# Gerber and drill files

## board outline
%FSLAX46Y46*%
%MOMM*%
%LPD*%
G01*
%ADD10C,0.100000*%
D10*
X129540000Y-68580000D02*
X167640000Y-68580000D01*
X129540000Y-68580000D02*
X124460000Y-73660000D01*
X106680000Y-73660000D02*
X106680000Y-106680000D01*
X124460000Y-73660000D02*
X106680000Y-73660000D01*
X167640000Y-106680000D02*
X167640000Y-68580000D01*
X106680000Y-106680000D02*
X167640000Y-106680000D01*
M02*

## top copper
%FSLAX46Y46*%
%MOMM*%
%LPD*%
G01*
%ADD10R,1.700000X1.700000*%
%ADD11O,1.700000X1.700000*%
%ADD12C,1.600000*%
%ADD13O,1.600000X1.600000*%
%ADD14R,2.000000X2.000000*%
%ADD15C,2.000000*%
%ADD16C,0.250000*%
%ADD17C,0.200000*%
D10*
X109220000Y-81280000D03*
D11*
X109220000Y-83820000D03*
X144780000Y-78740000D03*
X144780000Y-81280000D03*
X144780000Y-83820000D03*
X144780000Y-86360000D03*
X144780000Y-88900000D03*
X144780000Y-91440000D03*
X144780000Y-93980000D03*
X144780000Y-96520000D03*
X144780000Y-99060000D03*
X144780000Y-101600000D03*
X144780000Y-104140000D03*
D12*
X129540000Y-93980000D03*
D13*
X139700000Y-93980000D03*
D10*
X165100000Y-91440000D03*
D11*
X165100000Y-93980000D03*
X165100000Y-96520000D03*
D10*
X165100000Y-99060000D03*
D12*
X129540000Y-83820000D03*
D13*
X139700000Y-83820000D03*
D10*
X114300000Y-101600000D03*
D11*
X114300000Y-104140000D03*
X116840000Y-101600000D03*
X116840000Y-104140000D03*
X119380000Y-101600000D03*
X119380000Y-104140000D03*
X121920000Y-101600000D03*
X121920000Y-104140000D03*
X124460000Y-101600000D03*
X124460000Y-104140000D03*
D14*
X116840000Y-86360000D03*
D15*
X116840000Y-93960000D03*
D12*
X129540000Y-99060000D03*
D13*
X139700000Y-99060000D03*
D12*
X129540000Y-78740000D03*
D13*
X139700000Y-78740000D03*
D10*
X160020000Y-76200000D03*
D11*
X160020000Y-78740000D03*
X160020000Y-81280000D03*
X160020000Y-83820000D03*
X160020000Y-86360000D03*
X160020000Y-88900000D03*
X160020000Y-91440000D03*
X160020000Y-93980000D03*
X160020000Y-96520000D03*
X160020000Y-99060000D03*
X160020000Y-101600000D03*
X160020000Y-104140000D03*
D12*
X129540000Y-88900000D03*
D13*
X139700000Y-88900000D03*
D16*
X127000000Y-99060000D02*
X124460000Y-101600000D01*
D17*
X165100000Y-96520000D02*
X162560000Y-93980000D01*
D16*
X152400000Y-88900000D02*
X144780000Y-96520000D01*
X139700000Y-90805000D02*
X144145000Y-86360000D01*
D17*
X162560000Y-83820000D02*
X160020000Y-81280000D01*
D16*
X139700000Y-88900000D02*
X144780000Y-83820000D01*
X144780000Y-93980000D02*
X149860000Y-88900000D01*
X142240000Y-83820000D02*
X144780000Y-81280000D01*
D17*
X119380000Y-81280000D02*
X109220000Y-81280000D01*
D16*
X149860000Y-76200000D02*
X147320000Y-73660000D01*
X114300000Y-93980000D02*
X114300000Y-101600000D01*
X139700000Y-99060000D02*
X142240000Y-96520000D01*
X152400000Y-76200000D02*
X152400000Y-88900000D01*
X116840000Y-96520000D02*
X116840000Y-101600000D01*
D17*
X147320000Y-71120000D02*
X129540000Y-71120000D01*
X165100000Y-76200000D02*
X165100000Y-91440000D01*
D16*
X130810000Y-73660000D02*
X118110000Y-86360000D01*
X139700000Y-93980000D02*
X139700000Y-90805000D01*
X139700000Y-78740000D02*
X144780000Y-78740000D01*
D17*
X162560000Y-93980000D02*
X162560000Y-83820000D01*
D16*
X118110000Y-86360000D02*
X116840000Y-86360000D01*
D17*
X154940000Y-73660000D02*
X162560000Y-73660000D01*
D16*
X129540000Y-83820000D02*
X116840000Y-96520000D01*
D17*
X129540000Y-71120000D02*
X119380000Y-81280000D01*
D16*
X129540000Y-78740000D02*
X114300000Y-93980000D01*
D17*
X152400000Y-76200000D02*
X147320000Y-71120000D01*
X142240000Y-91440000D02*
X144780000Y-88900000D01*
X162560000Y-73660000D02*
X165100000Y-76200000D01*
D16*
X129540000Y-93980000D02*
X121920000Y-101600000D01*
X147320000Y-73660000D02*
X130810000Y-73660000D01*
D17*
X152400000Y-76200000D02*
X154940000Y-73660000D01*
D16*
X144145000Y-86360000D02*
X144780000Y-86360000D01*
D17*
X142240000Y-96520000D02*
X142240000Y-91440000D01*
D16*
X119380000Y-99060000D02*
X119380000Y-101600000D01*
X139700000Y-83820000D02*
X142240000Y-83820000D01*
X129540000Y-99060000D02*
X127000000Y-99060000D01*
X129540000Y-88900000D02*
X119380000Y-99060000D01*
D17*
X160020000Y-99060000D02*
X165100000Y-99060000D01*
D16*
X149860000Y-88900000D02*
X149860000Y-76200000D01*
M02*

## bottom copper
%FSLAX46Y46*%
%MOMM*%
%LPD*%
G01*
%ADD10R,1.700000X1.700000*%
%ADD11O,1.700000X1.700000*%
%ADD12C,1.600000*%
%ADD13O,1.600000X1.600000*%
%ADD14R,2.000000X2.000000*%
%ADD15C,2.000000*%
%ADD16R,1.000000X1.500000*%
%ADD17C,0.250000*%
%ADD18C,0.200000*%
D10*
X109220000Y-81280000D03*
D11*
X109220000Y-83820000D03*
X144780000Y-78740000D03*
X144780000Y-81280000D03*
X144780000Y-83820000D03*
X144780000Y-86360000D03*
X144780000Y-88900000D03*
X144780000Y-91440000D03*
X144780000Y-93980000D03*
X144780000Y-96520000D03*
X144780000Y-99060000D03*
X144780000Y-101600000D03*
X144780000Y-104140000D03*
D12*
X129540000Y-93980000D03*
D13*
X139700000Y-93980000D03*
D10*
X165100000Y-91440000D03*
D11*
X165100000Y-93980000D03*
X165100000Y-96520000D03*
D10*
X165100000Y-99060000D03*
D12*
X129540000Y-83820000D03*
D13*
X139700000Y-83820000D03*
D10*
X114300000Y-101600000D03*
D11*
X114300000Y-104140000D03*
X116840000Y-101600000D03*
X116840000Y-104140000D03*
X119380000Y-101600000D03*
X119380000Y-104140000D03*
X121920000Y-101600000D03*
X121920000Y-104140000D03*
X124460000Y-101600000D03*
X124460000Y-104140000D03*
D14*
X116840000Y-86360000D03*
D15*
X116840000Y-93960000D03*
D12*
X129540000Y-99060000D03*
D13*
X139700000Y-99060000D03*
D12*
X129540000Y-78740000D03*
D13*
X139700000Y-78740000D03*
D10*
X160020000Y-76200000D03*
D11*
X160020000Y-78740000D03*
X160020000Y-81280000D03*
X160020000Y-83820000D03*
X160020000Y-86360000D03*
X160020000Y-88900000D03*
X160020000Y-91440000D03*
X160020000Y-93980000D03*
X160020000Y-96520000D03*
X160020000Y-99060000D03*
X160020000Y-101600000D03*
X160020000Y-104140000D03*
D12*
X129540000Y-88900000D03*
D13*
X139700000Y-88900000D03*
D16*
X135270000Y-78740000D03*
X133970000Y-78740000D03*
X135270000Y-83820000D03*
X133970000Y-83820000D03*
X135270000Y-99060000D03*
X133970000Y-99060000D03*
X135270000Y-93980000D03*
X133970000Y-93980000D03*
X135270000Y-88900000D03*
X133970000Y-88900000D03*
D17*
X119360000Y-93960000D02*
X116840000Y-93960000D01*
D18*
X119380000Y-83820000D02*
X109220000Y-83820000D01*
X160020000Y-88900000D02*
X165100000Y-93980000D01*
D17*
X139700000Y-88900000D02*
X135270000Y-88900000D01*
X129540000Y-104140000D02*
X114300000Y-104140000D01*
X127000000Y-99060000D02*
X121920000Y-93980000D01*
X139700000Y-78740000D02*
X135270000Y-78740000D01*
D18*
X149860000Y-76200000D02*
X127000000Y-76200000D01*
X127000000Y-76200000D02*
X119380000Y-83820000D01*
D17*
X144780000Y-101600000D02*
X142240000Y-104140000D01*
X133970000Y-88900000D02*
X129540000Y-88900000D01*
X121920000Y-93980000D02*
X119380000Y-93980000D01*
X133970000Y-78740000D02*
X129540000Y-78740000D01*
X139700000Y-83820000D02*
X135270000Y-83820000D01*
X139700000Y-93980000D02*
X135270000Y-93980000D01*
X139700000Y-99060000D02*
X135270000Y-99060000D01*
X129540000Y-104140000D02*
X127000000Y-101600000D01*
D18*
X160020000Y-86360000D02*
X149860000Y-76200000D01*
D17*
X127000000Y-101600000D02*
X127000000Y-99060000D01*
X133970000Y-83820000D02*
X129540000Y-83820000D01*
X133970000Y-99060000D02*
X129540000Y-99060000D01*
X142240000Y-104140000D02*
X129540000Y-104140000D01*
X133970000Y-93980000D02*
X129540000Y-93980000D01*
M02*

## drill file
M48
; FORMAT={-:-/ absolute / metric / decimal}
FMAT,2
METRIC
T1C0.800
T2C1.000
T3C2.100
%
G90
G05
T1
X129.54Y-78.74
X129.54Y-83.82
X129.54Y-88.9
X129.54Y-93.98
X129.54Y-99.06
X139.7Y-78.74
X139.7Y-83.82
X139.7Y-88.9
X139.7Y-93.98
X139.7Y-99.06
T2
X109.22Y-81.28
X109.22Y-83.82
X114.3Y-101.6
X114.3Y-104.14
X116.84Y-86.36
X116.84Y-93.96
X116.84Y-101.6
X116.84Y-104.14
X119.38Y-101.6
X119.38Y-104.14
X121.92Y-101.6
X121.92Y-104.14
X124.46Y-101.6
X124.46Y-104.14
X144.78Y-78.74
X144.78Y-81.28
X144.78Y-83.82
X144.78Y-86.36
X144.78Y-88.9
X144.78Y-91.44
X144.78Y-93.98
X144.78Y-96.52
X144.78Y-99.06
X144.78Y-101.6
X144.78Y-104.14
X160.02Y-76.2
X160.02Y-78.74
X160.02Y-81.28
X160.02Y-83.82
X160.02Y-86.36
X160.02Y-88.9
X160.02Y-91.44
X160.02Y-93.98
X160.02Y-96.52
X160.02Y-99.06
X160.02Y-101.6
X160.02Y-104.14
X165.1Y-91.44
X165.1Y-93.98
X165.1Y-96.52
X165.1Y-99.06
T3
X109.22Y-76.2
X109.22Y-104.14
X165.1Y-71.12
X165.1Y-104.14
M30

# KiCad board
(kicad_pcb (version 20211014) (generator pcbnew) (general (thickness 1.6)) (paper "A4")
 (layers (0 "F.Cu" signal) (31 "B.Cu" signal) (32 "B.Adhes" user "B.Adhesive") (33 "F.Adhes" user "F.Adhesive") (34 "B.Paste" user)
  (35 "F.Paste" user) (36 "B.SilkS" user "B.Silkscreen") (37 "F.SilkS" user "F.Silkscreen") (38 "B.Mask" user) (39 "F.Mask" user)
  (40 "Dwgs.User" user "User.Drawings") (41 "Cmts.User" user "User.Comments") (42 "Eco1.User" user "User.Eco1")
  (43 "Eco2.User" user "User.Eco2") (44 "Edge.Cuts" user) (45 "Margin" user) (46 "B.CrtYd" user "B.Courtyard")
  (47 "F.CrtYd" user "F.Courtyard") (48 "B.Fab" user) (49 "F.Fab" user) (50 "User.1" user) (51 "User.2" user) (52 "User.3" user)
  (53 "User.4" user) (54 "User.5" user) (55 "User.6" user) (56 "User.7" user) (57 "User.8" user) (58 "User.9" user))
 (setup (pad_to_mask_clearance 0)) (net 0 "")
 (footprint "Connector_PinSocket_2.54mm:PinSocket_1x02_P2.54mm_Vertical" (layer "F.Cu") (at 109.22 81.28)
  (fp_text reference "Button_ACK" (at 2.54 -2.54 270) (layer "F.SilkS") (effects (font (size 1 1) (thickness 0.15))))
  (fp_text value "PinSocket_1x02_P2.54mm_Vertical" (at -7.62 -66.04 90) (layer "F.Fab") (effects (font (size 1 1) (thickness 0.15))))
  (pad "1" thru_hole rect (at 0 0) (size 1.7 1.7) (drill 1) (layers *.Cu *.Mask))
  (pad "2" thru_hole oval (at 0 2.54) (size 1.7 1.7) (drill 1) (layers *.Cu *.Mask)))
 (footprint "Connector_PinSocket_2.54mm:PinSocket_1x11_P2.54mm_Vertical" (layer "F.Cu") (at 144.78 78.74)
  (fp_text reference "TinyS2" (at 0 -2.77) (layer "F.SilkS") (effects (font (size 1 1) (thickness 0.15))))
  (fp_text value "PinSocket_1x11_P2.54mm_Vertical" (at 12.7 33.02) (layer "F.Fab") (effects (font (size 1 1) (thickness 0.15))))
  (pad "1" thru_hole oval (at 0 0) (size 1.7 1.7) (drill 1) (layers *.Cu *.Mask))
  (pad "2" thru_hole oval (at 0 2.54) (size 1.7 1.7) (drill 1) (layers *.Cu *.Mask))
  (pad "3" thru_hole oval (at 0 5.08) (size 1.7 1.7) (drill 1) (layers *.Cu *.Mask))
  (pad "4" thru_hole oval (at 0 7.62) (size 1.7 1.7) (drill 1) (layers *.Cu *.Mask))
  (pad "5" thru_hole oval (at 0 10.16) (size 1.7 1.7) (drill 1) (layers *.Cu *.Mask))
  (pad "6" thru_hole oval (at 0 12.7) (size 1.7 1.7) (drill 1) (layers *.Cu *.Mask))
  (pad "7" thru_hole oval (at 0 15.24) (size 1.7 1.7) (drill 1) (layers *.Cu *.Mask))
  (pad "8" thru_hole oval (at 0 17.78) (size 1.7 1.7) (drill 1) (layers *.Cu *.Mask))
  (pad "9" thru_hole oval (at 0 20.32) (size 1.7 1.7) (drill 1) (layers *.Cu *.Mask))
  (pad "10" thru_hole oval (at 0 22.86) (size 1.7 1.7) (drill 1) (layers *.Cu *.Mask))
  (pad "11" thru_hole oval (at 0 25.4) (size 1.7 1.7) (drill 1) (layers *.Cu *.Mask)))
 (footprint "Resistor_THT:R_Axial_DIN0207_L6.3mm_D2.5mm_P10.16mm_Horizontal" (layer "F.Cu") (at 129.54 93.98)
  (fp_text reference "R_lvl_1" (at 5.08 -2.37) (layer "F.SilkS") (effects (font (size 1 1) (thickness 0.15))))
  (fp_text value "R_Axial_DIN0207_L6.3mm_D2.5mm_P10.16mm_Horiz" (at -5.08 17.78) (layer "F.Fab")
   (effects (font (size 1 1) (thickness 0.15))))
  (pad "1" thru_hole circle (at 0 0) (size 1.6 1.6) (drill 0.8) (layers *.Cu *.Mask))
  (pad "2" thru_hole oval (at 10.16 0) (size 1.6 1.6) (drill 0.8) (layers *.Cu *.Mask)))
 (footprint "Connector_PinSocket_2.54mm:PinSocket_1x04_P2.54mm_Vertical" (layer "F.Cu") (at 165.1 91.44)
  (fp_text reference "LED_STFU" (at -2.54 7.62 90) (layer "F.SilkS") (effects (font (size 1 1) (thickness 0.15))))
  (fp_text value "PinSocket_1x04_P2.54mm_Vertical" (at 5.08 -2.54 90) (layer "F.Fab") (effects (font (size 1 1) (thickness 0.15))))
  (pad "1" thru_hole rect (at 0 0) (size 1.7 1.7) (drill 1) (layers *.Cu *.Mask))
  (pad "2" thru_hole oval (at 0 2.54) (size 1.7 1.7) (drill 1) (layers *.Cu *.Mask))
  (pad "3" thru_hole oval (at 0 5.08) (size 1.7 1.7) (drill 1) (layers *.Cu *.Mask))
  (pad "4" thru_hole rect (at 0 7.62) (size 1.7 1.7) (drill 1) (layers *.Cu *.Mask)))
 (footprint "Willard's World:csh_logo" (layer "F.Cu") (at 116.84 78.74)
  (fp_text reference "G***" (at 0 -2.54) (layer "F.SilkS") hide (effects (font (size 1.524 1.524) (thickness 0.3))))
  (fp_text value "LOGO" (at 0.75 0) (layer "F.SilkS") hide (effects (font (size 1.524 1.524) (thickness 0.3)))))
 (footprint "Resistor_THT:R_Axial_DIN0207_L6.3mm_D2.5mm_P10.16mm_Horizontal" (layer "F.Cu") (at 129.54 83.82)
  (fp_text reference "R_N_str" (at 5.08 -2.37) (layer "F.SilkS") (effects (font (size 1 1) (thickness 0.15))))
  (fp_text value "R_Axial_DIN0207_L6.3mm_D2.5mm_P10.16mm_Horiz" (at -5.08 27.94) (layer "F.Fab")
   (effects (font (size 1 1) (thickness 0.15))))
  (pad "1" thru_hole circle (at 0 0) (size 1.6 1.6) (drill 0.8) (layers *.Cu *.Mask))
  (pad "2" thru_hole oval (at 10.16 0) (size 1.6 1.6) (drill 0.8) (layers *.Cu *.Mask)))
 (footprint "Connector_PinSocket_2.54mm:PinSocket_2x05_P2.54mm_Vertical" (layer "F.Cu") (at 114.3 101.6 90)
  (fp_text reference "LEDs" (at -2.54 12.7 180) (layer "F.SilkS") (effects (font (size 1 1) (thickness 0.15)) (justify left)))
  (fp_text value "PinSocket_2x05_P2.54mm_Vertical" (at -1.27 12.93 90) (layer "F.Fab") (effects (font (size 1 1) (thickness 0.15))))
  (pad "1" thru_hole rect (at 0 0 90) (size 1.7 1.7) (drill 1) (layers *.Cu *.Mask))
  (pad "2" thru_hole oval (at -2.54 0 90) (size 1.7 1.7) (drill 1) (layers *.Cu *.Mask))
  (pad "3" thru_hole oval (at 0 2.54 90) (size 1.7 1.7) (drill 1) (layers *.Cu *.Mask))
  (pad "4" thru_hole oval (at -2.54 2.54 90) (size 1.7 1.7) (drill 1) (layers *.Cu *.Mask))
  (pad "5" thru_hole oval (at 0 5.08 90) (size 1.7 1.7) (drill 1) (layers *.Cu *.Mask))
  (pad "6" thru_hole oval (at -2.54 5.08 90) (size 1.7 1.7) (drill 1) (layers *.Cu *.Mask))
  (pad "7" thru_hole oval (at 0 7.62 90) (size 1.7 1.7) (drill 1) (layers *.Cu *.Mask))
  (pad "8" thru_hole oval (at -2.54 7.62 90) (size 1.7 1.7) (drill 1) (layers *.Cu *.Mask))
  (pad "9" thru_hole oval (at 0 10.16 90) (size 1.7 1.7) (drill 1) (layers *.Cu *.Mask))
  (pad "10" thru_hole oval (at -2.54 10.16 90) (size 1.7 1.7) (drill 1) (layers *.Cu *.Mask)))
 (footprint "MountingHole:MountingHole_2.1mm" (layer "F.Cu") (at 109.22 76.2)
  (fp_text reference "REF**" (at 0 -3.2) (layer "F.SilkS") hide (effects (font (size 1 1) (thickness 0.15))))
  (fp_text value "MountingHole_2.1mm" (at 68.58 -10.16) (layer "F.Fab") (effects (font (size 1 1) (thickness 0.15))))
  (pad "" np_thru_hole circle (at 0 0) (size 2.1 2.1) (drill 2.1) (layers *.Cu *.Mask)))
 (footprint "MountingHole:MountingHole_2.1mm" (layer "F.Cu") (at 109.22 104.14 90)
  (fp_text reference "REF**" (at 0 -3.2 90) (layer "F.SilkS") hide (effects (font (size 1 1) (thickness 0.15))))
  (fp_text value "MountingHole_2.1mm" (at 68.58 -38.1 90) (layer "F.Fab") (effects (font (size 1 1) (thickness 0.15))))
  (pad "" np_thru_hole circle (at 0 0 90) (size 2.1 2.1) (drill 2.1) (layers *.Cu *.Mask)))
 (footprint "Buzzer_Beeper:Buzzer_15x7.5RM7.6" (layer "F.Cu") (at 116.84 86.36 -90)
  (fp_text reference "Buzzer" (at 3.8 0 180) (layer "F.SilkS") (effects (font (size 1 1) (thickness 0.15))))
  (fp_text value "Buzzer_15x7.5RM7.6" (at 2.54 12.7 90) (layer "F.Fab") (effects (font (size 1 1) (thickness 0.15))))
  (pad "1" thru_hole rect (at 0 0 270) (size 2 2) (drill 1) (layers *.Cu *.Mask))
  (pad "2" thru_hole circle (at 7.6 0 270) (size 2 2) (drill 1) (layers *.Cu *.Mask)))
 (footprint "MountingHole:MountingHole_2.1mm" (layer "F.Cu") (at 165.1 71.12)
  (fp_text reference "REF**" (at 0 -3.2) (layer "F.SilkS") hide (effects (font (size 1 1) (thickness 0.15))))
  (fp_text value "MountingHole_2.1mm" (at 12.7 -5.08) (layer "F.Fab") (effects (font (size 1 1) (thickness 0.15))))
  (pad "" np_thru_hole circle (at 0 0) (size 2.1 2.1) (drill 2.1) (layers *.Cu *.Mask)))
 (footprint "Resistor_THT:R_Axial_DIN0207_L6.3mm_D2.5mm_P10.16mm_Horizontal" (layer "F.Cu") (at 129.54 99.06)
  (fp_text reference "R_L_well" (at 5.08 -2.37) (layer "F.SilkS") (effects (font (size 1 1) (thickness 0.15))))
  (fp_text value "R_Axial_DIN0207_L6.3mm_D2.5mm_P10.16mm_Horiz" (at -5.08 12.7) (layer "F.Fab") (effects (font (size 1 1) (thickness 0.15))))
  (pad "1" thru_hole circle (at 0 0) (size 1.6 1.6) (drill 0.8) (layers *.Cu *.Mask))
  (pad "2" thru_hole oval (at 10.16 0) (size 1.6 1.6) (drill 0.8) (layers *.Cu *.Mask)))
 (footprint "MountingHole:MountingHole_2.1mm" (layer "F.Cu") (at 165.1 104.14)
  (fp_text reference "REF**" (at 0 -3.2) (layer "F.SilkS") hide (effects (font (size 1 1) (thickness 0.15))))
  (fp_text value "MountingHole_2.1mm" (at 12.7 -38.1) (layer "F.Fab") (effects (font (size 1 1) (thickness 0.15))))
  (pad "" np_thru_hole circle (at 0 0) (size 2.1 2.1) (drill 2.1) (layers *.Cu *.Mask)))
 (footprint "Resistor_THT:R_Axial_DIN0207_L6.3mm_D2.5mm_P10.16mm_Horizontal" (layer "F.Cu") (at 129.54 78.74)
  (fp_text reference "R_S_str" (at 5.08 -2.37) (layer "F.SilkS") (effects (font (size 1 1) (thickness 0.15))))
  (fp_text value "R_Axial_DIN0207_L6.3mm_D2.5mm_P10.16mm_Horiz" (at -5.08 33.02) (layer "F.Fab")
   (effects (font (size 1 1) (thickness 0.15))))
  (pad "1" thru_hole circle (at 0 0) (size 1.6 1.6) (drill 0.8) (layers *.Cu *.Mask))
  (pad "2" thru_hole oval (at 10.16 0) (size 1.6 1.6) (drill 0.8) (layers *.Cu *.Mask)))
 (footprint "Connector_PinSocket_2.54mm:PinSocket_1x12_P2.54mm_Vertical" (layer "F.Cu") (at 160.02 76.2)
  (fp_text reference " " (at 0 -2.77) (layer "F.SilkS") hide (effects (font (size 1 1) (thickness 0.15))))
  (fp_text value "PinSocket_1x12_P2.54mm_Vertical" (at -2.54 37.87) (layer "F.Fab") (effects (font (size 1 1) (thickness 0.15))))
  (pad "1" thru_hole rect (at 0 0) (size 1.7 1.7) (drill 1) (layers *.Cu *.Mask))
  (pad "2" thru_hole oval (at 0 2.54) (size 1.7 1.7) (drill 1) (layers *.Cu *.Mask))
  (pad "3" thru_hole oval (at 0 5.08) (size 1.7 1.7) (drill 1) (layers *.Cu *.Mask))
  (pad "4" thru_hole oval (at 0 7.62) (size 1.7 1.7) (drill 1) (layers *.Cu *.Mask))
  (pad "5" thru_hole oval (at 0 10.16) (size 1.7 1.7) (drill 1) (layers *.Cu *.Mask))
  (pad "6" thru_hole oval (at 0 12.7) (size 1.7 1.7) (drill 1) (layers *.Cu *.Mask))
  (pad "7" thru_hole oval (at 0 15.24) (size 1.7 1.7) (drill 1) (layers *.Cu *.Mask))
  (pad "8" thru_hole oval (at 0 17.78) (size 1.7 1.7) (drill 1) (layers *.Cu *.Mask))
  (pad "9" thru_hole oval (at 0 20.32) (size 1.7 1.7) (drill 1) (layers *.Cu *.Mask))
  (pad "10" thru_hole oval (at 0 22.86) (size 1.7 1.7) (drill 1) (layers *.Cu *.Mask))
  (pad "11" thru_hole oval (at 0 25.4) (size 1.7 1.7) (drill 1) (layers *.Cu *.Mask))
  (pad "12" thru_hole oval (at 0 27.94) (size 1.7 1.7) (drill 1) (layers *.Cu *.Mask)))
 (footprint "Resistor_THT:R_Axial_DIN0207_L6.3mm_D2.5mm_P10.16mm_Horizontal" (layer "F.Cu") (at 129.54 88.9)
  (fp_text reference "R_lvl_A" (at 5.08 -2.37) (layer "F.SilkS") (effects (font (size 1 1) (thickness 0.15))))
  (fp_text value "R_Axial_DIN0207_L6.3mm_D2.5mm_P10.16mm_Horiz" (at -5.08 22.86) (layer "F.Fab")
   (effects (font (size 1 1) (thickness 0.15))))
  (pad "1" thru_hole circle (at 0 0) (size 1.6 1.6) (drill 0.8) (layers *.Cu *.Mask))
  (pad "2" thru_hole oval (at 10.16 0) (size 1.6 1.6) (drill 0.8) (layers *.Cu *.Mask)))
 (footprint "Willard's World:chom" (layer "B.Cu") (at 116.84 93.98 180)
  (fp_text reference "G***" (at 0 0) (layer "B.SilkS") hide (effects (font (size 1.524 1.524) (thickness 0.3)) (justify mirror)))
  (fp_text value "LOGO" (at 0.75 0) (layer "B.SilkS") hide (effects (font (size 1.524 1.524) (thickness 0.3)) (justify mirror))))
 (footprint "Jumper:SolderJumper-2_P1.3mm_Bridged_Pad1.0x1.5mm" (layer "B.Cu") (at 134.62 78.74 180)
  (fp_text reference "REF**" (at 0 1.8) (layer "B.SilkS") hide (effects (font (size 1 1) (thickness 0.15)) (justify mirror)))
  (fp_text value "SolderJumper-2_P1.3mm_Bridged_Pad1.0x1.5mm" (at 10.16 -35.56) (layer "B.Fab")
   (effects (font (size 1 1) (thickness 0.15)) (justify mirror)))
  (pad "1" smd rect (at -0.65 0 180) (size 1 1.5) (layers "B.Cu" "B.Mask"))
  (pad "2" smd rect (at 0.65 0 180) (size 1 1.5) (layers "B.Cu" "B.Mask")))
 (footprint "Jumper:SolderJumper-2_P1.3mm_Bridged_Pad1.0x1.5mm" (layer "B.Cu") (at 134.62 83.82 180)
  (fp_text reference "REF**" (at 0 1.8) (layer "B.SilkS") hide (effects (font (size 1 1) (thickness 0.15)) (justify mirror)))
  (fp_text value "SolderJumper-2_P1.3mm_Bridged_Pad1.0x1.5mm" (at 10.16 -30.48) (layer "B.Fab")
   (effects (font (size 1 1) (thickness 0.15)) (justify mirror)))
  (pad "1" smd rect (at -0.65 0 180) (size 1 1.5) (layers "B.Cu" "B.Mask"))
  (pad "2" smd rect (at 0.65 0 180) (size 1 1.5) (layers "B.Cu" "B.Mask")))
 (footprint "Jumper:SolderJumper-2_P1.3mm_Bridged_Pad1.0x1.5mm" (layer "B.Cu") (at 134.62 99.06 180)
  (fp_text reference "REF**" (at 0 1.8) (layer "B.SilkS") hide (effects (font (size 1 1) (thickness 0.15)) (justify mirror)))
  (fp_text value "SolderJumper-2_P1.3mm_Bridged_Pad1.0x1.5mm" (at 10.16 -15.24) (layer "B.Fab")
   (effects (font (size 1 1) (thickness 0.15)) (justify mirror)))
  (pad "1" smd rect (at -0.65 0 180) (size 1 1.5) (layers "B.Cu" "B.Mask"))
  (pad "2" smd rect (at 0.65 0 180) (size 1 1.5) (layers "B.Cu" "B.Mask")))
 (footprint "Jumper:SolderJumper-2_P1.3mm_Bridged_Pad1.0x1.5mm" (layer "B.Cu") (at 134.62 93.98 180)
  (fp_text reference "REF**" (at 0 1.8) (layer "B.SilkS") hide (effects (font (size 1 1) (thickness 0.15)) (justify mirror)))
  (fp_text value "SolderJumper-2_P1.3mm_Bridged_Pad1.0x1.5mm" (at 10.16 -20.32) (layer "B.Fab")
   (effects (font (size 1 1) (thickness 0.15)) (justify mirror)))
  (pad "1" smd rect (at -0.65 0 180) (size 1 1.5) (layers "B.Cu" "B.Mask"))
  (pad "2" smd rect (at 0.65 0 180) (size 1 1.5) (layers "B.Cu" "B.Mask")))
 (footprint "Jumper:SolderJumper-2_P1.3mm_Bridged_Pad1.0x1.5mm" (layer "B.Cu") (at 134.62 88.9 180)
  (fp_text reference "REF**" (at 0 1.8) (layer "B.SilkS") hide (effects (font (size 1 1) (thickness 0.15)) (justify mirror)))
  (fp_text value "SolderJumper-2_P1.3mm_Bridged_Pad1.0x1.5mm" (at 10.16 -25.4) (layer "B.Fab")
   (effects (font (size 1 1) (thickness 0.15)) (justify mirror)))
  (pad "1" smd rect (at -0.65 0 180) (size 1 1.5) (layers "B.Cu" "B.Mask"))
  (pad "2" smd rect (at 0.65 0 180) (size 1 1.5) (layers "B.Cu" "B.Mask")))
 (gr_line (start 129.54 68.58) (end 167.64 68.58) (layer "Edge.Cuts") (width 0.1))
 (gr_line (start 129.54 68.58) (end 124.46 73.66) (layer "Edge.Cuts") (width 0.1))
 (gr_line (start 106.68 73.66) (end 106.68 106.68) (layer "Edge.Cuts") (width 0.1))
 (gr_line (start 124.46 73.66) (end 106.68 73.66) (layer "Edge.Cuts") (width 0.1))
 (gr_line (start 167.64 106.68) (end 167.64 68.58) (layer "Edge.Cuts") (width 0.1))
 (gr_line (start 106.68 106.68) (end 167.64 106.68) (layer "Edge.Cuts") (width 0.1))
 (segment (start 127 99.06) (end 124.46 101.6) (width 0.25) (layer "F.Cu") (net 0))
 (segment (start 165.1 96.52) (end 162.56 93.98) (width 0.2) (layer "F.Cu") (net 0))
 (segment (start 152.4 88.9) (end 144.78 96.52) (width 0.25) (layer "F.Cu") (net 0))
 (segment (start 139.7 90.805) (end 144.145 86.36) (width 0.25) (layer "F.Cu") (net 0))
 (segment (start 162.56 83.82) (end 160.02 81.28) (width 0.2) (layer "F.Cu") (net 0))
 (segment (start 139.7 88.9) (end 144.78 83.82) (width 0.25) (layer "F.Cu") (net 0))
 (segment (start 144.78 93.98) (end 149.86 88.9) (width 0.25) (layer "F.Cu") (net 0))
 (segment (start 142.24 83.82) (end 144.78 81.28) (width 0.25) (layer "F.Cu") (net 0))
 (segment (start 119.38 81.28) (end 109.22 81.28) (width 0.2) (layer "F.Cu") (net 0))
 (segment (start 149.86 76.2) (end 147.32 73.66) (width 0.25) (layer "F.Cu") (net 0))
 (segment (start 114.3 93.98) (end 114.3 101.6) (width 0.25) (layer "F.Cu") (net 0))
 (segment (start 139.7 99.06) (end 142.24 96.52) (width 0.25) (layer "F.Cu") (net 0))
 (segment (start 152.4 76.2) (end 152.4 88.9) (width 0.25) (layer "F.Cu") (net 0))
 (segment (start 116.84 96.52) (end 116.84 101.6) (width 0.25) (layer "F.Cu") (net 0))
 (segment (start 147.32 71.12) (end 129.54 71.12) (width 0.2) (layer "F.Cu") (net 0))
 (segment (start 165.1 76.2) (end 165.1 91.44) (width 0.2) (layer "F.Cu") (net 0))
 (segment (start 130.81 73.66) (end 118.11 86.36) (width 0.25) (layer "F.Cu") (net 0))
 (segment (start 139.7 93.98) (end 139.7 90.805) (width 0.25) (layer "F.Cu") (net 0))
 (segment (start 139.7 78.74) (end 144.78 78.74) (width 0.25) (layer "F.Cu") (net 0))
 (segment (start 162.56 93.98) (end 162.56 83.82) (width 0.2) (layer "F.Cu") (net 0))
 (segment (start 118.11 86.36) (end 116.84 86.36) (width 0.25) (layer "F.Cu") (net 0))
 (segment (start 154.94 73.66) (end 162.56 73.66) (width 0.2) (layer "F.Cu") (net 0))
 (segment (start 129.54 83.82) (end 116.84 96.52) (width 0.25) (layer "F.Cu") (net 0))
 (segment (start 129.54 71.12) (end 119.38 81.28) (width 0.2) (layer "F.Cu") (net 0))
 (segment (start 129.54 78.74) (end 114.3 93.98) (width 0.25) (layer "F.Cu") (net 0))
 (segment (start 152.4 76.2) (end 147.32 71.12) (width 0.2) (layer "F.Cu") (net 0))
 (segment (start 142.24 91.44) (end 144.78 88.9) (width 0.2) (layer "F.Cu") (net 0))
 (segment (start 162.56 73.66) (end 165.1 76.2) (width 0.2) (layer "F.Cu") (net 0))
 (segment (start 129.54 93.98) (end 121.92 101.6) (width 0.25) (layer "F.Cu") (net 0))
 (segment (start 147.32 73.66) (end 130.81 73.66) (width 0.25) (layer "F.Cu") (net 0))
 (segment (start 152.4 76.2) (end 154.94 73.66) (width 0.2) (layer "F.Cu") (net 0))
 (segment (start 144.145 86.36) (end 144.78 86.36) (width 0.25) (layer "F.Cu") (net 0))
 (segment (start 142.24 96.52) (end 142.24 91.44) (width 0.2) (layer "F.Cu") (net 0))
 (segment (start 119.38 99.06) (end 119.38 101.6) (width 0.25) (layer "F.Cu") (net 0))
 (segment (start 139.7 83.82) (end 142.24 83.82) (width 0.25) (layer "F.Cu") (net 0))
 (segment (start 129.54 99.06) (end 127 99.06) (width 0.25) (layer "F.Cu") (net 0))
 (segment (start 129.54 88.9) (end 119.38 99.06) (width 0.25) (layer "F.Cu") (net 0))
 (segment (start 160.02 99.06) (end 165.1 99.06) (width 0.2) (layer "F.Cu") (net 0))
 (segment (start 149.86 88.9) (end 149.86 76.2) (width 0.25) (layer "F.Cu") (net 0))
 (segment (start 119.36 93.96) (end 116.84 93.96) (width 0.25) (layer "B.Cu") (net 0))
 (segment (start 119.38 83.82) (end 109.22 83.82) (width 0.2) (layer "B.Cu") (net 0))
 (segment (start 160.02 88.9) (end 165.1 93.98) (width 0.2) (layer "B.Cu") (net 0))
 (segment (start 139.7 88.9) (end 135.27 88.9) (width 0.25) (layer "B.Cu") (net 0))
 (segment (start 129.54 104.14) (end 114.3 104.14) (width 0.25) (layer "B.Cu") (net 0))
 (segment (start 127 99.06) (end 121.92 93.98) (width 0.25) (layer "B.Cu") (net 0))
 (segment (start 139.7 78.74) (end 135.27 78.74) (width 0.25) (layer "B.Cu") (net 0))
 (segment (start 149.86 76.2) (end 127 76.2) (width 0.2) (layer "B.Cu") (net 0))
 (segment (start 127 76.2) (end 119.38 83.82) (width 0.2) (layer "B.Cu") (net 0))
 (segment (start 144.78 101.6) (end 142.24 104.14) (width 0.25) (layer "B.Cu") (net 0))
 (segment (start 133.97 88.9) (end 129.54 88.9) (width 0.25) (layer "B.Cu") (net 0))
 (segment (start 121.92 93.98) (end 119.38 93.98) (width 0.25) (layer "B.Cu") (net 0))
 (segment (start 133.97 78.74) (end 129.54 78.74) (width 0.25) (layer "B.Cu") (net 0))
 (segment (start 139.7 83.82) (end 135.27 83.82) (width 0.25) (layer "B.Cu") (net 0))
 (segment (start 139.7 93.98) (end 135.27 93.98) (width 0.25) (layer "B.Cu") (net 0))
 (segment (start 139.7 99.06) (end 135.27 99.06) (width 0.25) (layer "B.Cu") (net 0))
 (segment (start 129.54 104.14) (end 127 101.6) (width 0.25) (layer "B.Cu") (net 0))
 (segment (start 160.02 86.36) (end 149.86 76.2) (width 0.2) (layer "B.Cu") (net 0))
 (segment (start 127 101.6) (end 127 99.06) (width 0.25) (layer "B.Cu") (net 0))
 (segment (start 133.97 83.82) (end 129.54 83.82) (width 0.25) (layer "B.Cu") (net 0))
 (segment (start 133.97 99.06) (end 129.54 99.06) (width 0.25) (layer "B.Cu") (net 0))
 (segment (start 142.24 104.14) (end 129.54 104.14) (width 0.25) (layer "B.Cu") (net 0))
 (segment (start 133.97 93.98) (end 129.54 93.98) (width 0.25) (layer "B.Cu") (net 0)))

